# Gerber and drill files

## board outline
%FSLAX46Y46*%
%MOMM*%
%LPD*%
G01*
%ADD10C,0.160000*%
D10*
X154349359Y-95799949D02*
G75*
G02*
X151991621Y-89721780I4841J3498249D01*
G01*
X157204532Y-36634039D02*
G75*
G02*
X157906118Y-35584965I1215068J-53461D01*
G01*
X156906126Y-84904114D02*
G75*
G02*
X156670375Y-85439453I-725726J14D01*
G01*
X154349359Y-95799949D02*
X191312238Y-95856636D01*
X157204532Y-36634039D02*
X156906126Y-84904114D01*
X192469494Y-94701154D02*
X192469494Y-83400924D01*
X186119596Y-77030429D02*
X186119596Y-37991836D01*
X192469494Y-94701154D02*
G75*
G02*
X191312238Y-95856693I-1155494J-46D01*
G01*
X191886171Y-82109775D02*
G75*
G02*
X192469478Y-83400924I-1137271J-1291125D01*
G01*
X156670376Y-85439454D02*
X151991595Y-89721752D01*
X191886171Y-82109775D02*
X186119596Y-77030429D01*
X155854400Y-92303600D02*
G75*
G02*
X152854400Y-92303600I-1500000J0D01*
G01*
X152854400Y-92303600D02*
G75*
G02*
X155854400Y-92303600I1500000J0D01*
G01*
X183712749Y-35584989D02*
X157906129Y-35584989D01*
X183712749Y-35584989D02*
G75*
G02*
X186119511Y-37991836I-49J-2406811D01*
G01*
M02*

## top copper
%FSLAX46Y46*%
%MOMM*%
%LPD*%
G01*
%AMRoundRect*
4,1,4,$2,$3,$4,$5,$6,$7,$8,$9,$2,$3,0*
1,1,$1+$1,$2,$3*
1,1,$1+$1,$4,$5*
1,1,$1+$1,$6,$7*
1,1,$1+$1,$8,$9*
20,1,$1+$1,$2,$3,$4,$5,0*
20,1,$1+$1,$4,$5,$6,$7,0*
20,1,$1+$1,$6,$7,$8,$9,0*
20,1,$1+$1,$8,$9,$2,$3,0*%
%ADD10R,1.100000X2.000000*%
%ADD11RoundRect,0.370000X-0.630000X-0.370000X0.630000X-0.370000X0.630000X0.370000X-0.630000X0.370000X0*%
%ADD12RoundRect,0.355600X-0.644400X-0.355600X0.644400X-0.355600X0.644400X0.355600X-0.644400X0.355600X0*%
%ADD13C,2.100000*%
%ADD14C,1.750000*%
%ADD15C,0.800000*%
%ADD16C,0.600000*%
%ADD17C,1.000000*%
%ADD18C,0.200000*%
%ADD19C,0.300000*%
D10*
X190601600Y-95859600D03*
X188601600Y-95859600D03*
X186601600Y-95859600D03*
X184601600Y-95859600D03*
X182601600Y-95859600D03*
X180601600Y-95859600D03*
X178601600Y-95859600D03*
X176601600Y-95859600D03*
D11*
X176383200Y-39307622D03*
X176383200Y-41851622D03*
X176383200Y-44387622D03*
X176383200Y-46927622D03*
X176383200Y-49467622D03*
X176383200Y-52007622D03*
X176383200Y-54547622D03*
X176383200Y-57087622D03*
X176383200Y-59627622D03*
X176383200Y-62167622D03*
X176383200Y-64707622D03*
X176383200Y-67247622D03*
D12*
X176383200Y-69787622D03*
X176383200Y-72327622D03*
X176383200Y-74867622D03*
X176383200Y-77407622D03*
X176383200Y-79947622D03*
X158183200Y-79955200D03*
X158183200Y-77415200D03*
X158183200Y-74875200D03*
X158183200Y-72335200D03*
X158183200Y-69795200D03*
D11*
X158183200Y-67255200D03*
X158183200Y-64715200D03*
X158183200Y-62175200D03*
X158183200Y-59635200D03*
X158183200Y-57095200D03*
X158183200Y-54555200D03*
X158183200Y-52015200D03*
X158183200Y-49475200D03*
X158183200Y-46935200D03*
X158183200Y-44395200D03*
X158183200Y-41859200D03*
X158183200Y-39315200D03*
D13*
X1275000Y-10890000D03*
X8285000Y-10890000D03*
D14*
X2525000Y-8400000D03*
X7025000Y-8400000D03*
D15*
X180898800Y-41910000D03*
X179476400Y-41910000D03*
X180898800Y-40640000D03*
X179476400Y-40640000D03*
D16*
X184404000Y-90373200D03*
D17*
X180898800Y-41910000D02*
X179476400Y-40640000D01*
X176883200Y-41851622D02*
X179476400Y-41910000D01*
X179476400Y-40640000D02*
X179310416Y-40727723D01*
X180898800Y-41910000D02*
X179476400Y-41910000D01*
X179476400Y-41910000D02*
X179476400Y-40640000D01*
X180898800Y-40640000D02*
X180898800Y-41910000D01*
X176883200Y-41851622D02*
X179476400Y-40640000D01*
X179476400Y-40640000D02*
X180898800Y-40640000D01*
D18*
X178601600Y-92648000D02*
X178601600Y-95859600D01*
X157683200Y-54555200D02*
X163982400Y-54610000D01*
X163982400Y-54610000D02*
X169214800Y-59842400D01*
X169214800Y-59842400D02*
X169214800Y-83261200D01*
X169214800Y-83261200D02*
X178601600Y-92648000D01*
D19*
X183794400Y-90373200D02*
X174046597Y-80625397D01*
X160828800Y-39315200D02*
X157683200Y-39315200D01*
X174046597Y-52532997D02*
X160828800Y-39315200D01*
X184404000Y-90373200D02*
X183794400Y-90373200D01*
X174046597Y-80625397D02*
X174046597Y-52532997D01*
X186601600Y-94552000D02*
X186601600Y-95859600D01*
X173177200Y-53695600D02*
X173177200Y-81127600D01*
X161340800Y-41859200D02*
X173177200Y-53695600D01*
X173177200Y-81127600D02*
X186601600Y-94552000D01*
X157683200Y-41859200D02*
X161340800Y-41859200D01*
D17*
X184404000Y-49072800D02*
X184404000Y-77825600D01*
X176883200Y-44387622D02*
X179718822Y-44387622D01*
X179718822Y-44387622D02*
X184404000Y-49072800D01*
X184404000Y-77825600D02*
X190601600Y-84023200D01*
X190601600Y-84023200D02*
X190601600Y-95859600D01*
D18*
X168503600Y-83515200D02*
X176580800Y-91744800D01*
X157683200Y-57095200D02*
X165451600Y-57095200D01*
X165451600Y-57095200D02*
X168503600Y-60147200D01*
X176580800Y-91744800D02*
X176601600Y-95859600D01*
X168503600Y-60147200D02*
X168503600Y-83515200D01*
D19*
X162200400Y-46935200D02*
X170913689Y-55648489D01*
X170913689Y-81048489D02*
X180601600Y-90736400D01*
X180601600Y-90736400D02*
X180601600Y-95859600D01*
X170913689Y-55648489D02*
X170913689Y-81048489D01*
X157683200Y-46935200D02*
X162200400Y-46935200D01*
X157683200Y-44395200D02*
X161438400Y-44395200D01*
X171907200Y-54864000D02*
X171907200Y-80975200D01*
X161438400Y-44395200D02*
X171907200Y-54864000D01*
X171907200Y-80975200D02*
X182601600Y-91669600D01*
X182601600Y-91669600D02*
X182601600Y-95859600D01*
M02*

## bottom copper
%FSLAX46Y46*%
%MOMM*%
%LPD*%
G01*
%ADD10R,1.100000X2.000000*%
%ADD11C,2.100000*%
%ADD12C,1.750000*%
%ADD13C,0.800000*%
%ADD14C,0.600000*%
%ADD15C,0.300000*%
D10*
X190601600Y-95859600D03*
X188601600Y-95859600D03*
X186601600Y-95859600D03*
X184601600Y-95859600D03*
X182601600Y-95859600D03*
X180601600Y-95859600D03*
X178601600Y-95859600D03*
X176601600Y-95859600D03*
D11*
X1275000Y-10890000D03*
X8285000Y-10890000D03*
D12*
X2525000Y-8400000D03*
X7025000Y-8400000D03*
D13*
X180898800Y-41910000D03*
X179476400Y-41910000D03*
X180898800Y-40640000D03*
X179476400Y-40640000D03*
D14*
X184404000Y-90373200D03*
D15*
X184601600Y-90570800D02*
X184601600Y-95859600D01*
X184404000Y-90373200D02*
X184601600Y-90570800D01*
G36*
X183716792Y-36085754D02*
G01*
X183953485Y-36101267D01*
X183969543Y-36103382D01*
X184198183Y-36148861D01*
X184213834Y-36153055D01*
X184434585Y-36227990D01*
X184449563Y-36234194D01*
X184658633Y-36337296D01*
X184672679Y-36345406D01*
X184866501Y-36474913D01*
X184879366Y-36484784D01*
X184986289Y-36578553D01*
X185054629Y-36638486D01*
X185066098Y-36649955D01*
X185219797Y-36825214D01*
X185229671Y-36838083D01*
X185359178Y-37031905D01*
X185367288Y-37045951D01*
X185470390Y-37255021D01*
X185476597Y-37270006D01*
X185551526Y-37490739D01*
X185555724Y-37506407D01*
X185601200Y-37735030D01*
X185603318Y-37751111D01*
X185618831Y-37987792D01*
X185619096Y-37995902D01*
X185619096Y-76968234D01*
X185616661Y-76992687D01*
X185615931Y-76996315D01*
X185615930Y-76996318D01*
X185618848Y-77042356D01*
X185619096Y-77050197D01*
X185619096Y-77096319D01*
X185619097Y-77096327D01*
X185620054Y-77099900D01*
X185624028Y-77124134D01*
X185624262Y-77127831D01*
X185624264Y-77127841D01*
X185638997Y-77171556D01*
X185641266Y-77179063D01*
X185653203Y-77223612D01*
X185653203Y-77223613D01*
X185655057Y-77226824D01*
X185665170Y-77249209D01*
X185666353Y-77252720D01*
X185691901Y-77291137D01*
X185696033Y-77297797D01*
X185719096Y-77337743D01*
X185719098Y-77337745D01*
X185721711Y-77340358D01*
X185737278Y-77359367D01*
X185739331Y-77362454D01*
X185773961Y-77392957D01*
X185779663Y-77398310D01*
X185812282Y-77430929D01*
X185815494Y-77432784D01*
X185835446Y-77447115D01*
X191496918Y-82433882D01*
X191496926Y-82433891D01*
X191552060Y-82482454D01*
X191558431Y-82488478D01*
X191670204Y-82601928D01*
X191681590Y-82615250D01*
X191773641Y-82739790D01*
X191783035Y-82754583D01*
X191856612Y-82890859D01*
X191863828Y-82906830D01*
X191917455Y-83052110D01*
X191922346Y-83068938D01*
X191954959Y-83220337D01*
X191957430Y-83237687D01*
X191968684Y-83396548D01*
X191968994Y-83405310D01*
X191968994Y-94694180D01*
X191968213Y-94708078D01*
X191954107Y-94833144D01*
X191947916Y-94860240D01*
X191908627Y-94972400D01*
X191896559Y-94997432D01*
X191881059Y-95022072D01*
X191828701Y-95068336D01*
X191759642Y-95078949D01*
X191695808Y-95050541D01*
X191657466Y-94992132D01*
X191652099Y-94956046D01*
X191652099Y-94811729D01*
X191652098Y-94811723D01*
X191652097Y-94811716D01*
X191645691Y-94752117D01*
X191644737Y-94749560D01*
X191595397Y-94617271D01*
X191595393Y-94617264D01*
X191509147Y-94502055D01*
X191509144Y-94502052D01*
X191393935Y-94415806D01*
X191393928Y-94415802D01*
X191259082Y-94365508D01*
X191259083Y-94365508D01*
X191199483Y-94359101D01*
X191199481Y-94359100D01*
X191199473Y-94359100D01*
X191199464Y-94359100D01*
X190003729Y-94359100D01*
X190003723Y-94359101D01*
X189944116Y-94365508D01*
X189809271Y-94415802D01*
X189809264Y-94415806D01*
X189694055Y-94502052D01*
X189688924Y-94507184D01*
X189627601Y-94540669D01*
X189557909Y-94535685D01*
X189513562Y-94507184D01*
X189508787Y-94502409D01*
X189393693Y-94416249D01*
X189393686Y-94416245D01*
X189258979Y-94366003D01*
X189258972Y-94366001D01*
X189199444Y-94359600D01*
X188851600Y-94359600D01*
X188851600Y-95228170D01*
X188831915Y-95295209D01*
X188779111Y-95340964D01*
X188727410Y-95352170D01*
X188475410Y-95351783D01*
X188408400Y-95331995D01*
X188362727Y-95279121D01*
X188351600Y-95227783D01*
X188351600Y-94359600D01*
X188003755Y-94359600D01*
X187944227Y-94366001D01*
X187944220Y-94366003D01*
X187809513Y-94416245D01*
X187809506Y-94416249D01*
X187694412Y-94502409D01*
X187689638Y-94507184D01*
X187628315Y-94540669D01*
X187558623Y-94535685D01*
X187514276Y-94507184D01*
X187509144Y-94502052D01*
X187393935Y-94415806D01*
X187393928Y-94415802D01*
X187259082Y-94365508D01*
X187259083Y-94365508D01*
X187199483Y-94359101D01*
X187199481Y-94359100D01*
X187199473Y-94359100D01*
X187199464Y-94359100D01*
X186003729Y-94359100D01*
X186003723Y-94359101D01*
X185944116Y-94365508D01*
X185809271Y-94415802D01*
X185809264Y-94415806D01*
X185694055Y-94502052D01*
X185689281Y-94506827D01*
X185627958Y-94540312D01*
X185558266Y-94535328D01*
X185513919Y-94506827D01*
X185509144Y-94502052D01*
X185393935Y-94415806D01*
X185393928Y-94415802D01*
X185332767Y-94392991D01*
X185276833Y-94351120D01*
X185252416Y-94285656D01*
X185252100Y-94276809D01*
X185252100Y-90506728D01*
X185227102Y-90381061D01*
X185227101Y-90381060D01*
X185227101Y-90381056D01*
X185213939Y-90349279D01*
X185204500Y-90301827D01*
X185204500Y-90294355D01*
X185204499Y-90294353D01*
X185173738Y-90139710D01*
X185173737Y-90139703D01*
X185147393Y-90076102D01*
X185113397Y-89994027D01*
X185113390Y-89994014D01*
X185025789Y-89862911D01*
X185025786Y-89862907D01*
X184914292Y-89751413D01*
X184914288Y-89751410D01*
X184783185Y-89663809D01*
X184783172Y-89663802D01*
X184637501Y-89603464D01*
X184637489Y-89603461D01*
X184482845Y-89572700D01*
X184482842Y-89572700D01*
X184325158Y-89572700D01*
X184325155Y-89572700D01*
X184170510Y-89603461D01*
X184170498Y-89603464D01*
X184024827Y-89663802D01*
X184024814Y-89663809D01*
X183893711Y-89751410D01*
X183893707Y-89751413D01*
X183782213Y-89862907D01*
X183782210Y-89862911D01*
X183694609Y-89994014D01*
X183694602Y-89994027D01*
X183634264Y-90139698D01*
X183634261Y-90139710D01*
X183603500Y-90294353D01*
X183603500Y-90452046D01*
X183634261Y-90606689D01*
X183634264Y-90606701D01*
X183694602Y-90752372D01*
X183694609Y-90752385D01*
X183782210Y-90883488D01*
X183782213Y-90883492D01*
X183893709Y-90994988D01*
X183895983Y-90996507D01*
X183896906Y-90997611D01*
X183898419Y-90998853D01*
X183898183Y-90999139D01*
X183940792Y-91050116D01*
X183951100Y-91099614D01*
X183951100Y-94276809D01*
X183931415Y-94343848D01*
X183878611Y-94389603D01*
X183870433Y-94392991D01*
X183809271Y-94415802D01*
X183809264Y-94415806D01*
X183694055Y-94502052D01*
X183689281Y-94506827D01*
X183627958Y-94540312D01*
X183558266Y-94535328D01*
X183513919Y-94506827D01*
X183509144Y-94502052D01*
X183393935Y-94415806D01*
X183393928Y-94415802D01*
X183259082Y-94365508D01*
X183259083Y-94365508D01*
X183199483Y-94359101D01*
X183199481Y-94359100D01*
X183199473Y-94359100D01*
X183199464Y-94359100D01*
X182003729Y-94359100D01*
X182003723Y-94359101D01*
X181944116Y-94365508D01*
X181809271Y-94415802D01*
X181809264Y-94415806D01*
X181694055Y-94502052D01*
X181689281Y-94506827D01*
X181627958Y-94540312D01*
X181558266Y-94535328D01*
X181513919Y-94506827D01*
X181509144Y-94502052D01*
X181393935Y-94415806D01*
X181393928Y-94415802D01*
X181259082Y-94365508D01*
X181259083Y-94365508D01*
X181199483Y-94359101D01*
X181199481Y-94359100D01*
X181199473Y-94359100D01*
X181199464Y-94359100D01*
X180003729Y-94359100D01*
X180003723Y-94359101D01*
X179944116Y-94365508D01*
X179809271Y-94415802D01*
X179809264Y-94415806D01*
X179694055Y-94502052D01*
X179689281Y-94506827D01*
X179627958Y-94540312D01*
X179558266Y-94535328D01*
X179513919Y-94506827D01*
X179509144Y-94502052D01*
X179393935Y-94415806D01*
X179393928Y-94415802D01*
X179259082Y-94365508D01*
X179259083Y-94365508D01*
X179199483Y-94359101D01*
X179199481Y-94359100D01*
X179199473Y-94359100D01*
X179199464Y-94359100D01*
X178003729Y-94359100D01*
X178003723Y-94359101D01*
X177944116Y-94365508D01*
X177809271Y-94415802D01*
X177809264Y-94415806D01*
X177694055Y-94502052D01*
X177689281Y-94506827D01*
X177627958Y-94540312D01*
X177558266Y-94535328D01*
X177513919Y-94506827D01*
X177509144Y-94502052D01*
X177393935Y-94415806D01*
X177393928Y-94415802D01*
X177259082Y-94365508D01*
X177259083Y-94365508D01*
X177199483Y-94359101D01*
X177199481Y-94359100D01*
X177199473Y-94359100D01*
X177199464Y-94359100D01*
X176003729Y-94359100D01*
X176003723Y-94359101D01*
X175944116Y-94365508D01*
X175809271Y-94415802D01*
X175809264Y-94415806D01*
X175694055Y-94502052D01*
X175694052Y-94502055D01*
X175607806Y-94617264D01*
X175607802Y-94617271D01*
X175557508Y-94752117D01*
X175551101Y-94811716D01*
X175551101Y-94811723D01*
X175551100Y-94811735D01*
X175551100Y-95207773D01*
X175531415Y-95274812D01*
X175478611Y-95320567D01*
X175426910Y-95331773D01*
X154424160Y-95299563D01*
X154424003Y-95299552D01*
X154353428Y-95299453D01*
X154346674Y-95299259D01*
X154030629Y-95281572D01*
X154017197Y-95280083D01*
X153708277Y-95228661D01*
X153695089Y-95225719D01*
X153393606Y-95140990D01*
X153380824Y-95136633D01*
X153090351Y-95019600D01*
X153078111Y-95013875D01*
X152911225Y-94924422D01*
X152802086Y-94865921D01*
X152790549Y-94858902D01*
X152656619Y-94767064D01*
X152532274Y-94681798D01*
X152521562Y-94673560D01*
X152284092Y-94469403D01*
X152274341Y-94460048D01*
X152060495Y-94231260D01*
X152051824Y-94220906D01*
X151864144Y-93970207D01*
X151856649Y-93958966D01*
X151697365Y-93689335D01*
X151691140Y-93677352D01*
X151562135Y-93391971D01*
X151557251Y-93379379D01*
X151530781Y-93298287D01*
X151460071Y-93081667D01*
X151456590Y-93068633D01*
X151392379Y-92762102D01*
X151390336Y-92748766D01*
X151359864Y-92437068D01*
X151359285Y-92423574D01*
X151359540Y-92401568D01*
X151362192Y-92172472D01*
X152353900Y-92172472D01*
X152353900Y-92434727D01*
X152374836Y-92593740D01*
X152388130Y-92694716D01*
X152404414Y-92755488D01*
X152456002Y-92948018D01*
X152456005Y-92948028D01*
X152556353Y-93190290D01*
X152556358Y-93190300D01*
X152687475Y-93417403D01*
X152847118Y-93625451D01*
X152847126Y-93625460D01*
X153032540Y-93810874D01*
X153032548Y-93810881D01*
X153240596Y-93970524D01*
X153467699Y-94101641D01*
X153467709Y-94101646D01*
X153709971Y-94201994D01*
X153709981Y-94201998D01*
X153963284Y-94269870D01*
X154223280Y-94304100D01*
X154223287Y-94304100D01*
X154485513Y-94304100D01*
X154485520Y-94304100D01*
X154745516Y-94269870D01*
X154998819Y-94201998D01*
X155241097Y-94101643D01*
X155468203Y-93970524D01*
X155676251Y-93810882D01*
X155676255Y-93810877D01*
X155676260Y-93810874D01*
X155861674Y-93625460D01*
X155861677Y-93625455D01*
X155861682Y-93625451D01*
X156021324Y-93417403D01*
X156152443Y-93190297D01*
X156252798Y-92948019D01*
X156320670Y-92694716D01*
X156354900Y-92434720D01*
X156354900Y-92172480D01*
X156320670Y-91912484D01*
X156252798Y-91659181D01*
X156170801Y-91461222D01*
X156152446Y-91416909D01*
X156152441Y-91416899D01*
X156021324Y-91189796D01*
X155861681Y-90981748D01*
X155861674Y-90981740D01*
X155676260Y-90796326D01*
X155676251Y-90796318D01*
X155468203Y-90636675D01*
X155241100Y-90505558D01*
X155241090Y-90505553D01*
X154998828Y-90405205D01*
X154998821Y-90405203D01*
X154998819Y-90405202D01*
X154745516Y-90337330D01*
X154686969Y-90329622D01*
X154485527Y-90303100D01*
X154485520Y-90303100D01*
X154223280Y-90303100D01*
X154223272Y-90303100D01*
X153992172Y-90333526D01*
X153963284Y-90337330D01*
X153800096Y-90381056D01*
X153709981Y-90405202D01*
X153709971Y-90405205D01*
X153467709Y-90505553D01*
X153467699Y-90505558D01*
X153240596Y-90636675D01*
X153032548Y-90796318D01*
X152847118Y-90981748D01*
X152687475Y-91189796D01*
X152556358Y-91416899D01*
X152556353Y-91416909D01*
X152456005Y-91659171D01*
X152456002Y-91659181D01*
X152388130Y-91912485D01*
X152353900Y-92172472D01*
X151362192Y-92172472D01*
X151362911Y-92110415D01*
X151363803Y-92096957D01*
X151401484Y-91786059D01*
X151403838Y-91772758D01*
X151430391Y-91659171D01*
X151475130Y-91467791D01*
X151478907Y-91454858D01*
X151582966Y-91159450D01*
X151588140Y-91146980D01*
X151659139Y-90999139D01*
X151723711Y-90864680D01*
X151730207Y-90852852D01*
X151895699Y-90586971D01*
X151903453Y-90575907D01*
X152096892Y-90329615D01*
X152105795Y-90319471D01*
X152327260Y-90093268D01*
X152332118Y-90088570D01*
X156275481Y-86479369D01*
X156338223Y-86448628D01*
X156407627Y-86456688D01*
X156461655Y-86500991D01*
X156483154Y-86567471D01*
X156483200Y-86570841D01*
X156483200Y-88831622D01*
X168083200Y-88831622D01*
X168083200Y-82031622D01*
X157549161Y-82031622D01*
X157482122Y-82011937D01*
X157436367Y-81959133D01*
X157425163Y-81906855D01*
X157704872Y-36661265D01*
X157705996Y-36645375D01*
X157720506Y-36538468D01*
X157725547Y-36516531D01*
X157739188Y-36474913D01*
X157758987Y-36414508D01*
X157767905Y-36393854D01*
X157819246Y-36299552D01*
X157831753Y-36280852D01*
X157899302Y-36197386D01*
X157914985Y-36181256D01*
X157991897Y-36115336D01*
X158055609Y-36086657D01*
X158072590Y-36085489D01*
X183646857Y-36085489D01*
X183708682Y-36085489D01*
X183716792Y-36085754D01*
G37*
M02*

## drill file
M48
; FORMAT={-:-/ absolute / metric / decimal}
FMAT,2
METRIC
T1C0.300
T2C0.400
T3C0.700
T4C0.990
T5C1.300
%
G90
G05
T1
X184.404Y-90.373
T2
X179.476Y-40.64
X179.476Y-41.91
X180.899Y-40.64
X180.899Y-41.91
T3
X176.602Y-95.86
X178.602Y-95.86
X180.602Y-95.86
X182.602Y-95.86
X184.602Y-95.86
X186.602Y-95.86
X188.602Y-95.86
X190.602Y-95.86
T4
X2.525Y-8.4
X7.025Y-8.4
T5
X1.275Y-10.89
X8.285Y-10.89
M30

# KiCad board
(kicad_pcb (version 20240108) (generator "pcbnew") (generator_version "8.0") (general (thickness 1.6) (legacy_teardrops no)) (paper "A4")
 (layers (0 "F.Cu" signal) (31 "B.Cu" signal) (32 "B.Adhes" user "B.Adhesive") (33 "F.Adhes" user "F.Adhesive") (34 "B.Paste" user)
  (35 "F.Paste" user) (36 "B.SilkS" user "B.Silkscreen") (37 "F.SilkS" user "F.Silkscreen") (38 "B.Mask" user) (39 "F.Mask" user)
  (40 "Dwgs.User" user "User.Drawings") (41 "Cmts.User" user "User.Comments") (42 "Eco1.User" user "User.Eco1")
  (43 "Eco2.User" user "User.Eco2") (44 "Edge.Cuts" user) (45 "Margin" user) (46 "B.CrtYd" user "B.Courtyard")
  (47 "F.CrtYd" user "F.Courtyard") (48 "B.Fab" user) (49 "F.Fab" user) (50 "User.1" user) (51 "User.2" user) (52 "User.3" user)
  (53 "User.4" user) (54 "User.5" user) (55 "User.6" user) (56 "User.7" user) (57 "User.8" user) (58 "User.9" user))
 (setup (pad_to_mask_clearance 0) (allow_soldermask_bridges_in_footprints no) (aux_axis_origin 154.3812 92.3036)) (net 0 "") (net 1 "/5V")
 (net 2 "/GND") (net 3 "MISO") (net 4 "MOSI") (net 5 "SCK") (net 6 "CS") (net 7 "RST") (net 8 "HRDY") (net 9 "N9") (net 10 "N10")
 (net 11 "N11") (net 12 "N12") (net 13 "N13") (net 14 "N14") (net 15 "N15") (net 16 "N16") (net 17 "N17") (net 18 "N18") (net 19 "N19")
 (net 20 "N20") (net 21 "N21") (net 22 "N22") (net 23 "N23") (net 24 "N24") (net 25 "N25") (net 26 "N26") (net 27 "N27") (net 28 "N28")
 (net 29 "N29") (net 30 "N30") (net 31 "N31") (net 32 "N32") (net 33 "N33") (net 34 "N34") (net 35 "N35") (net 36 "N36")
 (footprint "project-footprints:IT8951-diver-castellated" (layer "F.Cu") (at 183.6016 95.8596 180)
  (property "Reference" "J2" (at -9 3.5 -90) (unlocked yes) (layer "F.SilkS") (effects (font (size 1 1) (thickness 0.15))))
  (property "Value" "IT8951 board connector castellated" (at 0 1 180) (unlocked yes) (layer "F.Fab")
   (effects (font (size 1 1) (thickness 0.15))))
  (pad "1" thru_hole rect (at -7 0 180) (size 1.1 2) (drill 0.7) (layers "*.Cu" "*.Mask") (remove_unused_layers no) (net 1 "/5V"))
  (pad "2" thru_hole rect (at -5 0 180) (size 1.1 2) (drill 0.7) (layers "*.Cu" "*.Mask") (remove_unused_layers no) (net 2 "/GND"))
  (pad "3" thru_hole rect (at -3 0 180) (size 1.1 2) (drill 0.7) (layers "*.Cu" "*.Mask") (remove_unused_layers no) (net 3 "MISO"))
  (pad "4" thru_hole rect (at -1 0 180) (size 1.1 2) (drill 0.7) (layers "*.Cu" "*.Mask") (remove_unused_layers no) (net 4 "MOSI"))
  (pad "5" thru_hole rect (at 1 0 180) (size 1.1 2) (drill 0.7) (layers "*.Cu" "*.Mask") (remove_unused_layers no) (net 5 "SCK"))
  (pad "6" thru_hole rect (at 3 0 180) (size 1.1 2) (drill 0.7) (layers "*.Cu" "*.Mask") (remove_unused_layers no) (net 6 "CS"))
  (pad "7" thru_hole rect (at 5 0 180) (size 1.1 2) (drill 0.7) (layers "*.Cu" "*.Mask") (remove_unused_layers no) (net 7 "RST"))
  (pad "8" thru_hole rect (at 7 0 180) (size 1.1 2) (drill 0.7) (layers "*.Cu" "*.Mask") (remove_unused_layers no) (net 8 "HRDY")))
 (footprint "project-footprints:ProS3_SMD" (layer "F.Cu") (at 167.2832 60.831622)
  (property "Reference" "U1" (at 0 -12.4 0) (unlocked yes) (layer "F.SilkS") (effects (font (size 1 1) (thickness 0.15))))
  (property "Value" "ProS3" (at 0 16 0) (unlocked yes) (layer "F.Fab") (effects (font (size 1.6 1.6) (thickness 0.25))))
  (pad "1" smd roundrect (at 9.6 -21.524) (size 2 1.48) (drill (offset -0.5 0)) (layers "F.Cu" "F.Paste" "F.Mask") (roundrect_rratio 0.25)
   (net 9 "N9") (solder_mask_margin 0.0254))
  (pad "2" smd roundrect (at 9.6 -18.98) (size 2 1.48) (drill (offset -0.5 0)) (layers "F.Cu" "F.Paste" "F.Mask") (roundrect_rratio 0.25)
   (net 2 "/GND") (solder_mask_margin 0.0254))
  (pad "3" smd roundrect (at 9.6 -16.444) (size 2 1.48) (drill (offset -0.5 0)) (layers "F.Cu" "F.Paste" "F.Mask") (roundrect_rratio 0.25)
   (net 1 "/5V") (solder_mask_margin 0.0254))
  (pad "4" smd roundrect (at 9.6 -13.904) (size 2 1.48) (drill (offset -0.5 0)) (layers "F.Cu" "F.Paste" "F.Mask") (roundrect_rratio 0.25)
   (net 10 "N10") (solder_mask_margin 0.0254))
  (pad "5" smd roundrect (at 9.6 -11.364) (size 2 1.48) (drill (offset -0.5 0)) (layers "F.Cu" "F.Paste" "F.Mask") (roundrect_rratio 0.25)
   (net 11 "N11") (solder_mask_margin 0.0254))
  (pad "6" smd roundrect (at 9.6 -8.824) (size 2 1.48) (drill (offset -0.5 0)) (layers "F.Cu" "F.Paste" "F.Mask") (roundrect_rratio 0.25)
   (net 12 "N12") (solder_mask_margin 0.0254))
  (pad "7" smd roundrect (at 9.6 -6.284) (size 2 1.48) (drill (offset -0.5 0)) (layers "F.Cu" "F.Paste" "F.Mask") (roundrect_rratio 0.25)
   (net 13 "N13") (solder_mask_margin 0.0254))
  (pad "8" smd roundrect (at 9.6 -3.744) (size 2 1.48) (drill (offset -0.5 0)) (layers "F.Cu" "F.Paste" "F.Mask") (roundrect_rratio 0.25)
   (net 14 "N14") (solder_mask_margin 0.0254))
  (pad "9" smd roundrect (at 9.6 -1.204) (size 2 1.48) (drill (offset -0.5 0)) (layers "F.Cu" "F.Paste" "F.Mask") (roundrect_rratio 0.25)
   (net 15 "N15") (solder_mask_margin 0.0254))
  (pad "10" smd roundrect (at 9.6 1.336) (size 2 1.48) (drill (offset -0.5 0)) (layers "F.Cu" "F.Paste" "F.Mask") (roundrect_rratio 0.25)
   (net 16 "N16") (solder_mask_margin 0.0254))
  (pad "11" smd roundrect (at 9.6 3.876) (size 2 1.48) (drill (offset -0.5 0)) (layers "F.Cu" "F.Paste" "F.Mask") (roundrect_rratio 0.25)
   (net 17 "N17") (solder_mask_margin 0.0254))
  (pad "12" smd roundrect (at 9.6 6.416) (size 2 1.48) (drill (offset -0.5 0)) (layers "F.Cu" "F.Paste" "F.Mask") (roundrect_rratio 0.25)
   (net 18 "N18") (solder_mask_margin 0.0254))
  (pad "13" smd roundrect (at 9.6 8.956) (size 2 1.4224) (drill (offset -0.5 0)) (layers "F.Cu" "F.Paste" "F.Mask") (roundrect_rratio 0.25)
   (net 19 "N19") (solder_mask_margin 0.0254))
  (pad "14" smd roundrect (at 9.6 11.496) (size 2 1.4224) (drill (offset -0.5 0)) (layers "F.Cu" "F.Paste" "F.Mask") (roundrect_rratio 0.25)
   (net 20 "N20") (solder_mask_margin 0.0254))
  (pad "15" smd roundrect (at 9.6 14.036) (size 2 1.4224) (drill (offset -0.5 0)) (layers "F.Cu" "F.Paste" "F.Mask") (roundrect_rratio 0.25)
   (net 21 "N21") (solder_mask_margin 0.0254))
  (pad "16" smd roundrect (at 9.6 16.576) (size 2 1.4224) (drill (offset -0.5 0)) (layers "F.Cu" "F.Paste" "F.Mask") (roundrect_rratio 0.25)
   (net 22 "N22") (solder_mask_margin 0.0254))
  (pad "17" smd roundrect (at 9.6 19.116) (size 2 1.4224) (drill (offset -0.5 0)) (layers "F.Cu" "F.Paste" "F.Mask") (roundrect_rratio 0.25)
   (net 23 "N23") (solder_mask_margin 0.0254))
  (pad "18" smd roundrect (at -9.6 19.123578) (size 2 1.4224) (drill (offset 0.5 0)) (layers "F.Cu" "F.Paste" "F.Mask")
   (roundrect_rratio 0.25) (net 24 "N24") (solder_mask_margin 0.0254))
  (pad "19" smd roundrect (at -9.6 16.583578) (size 2 1.4224) (drill (offset 0.5 0)) (layers "F.Cu" "F.Paste" "F.Mask")
   (roundrect_rratio 0.25) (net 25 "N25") (solder_mask_margin 0.0254))
  (pad "20" smd roundrect (at -9.6 14.043578) (size 2 1.4224) (drill (offset 0.5 0)) (layers "F.Cu" "F.Paste" "F.Mask")
   (roundrect_rratio 0.25) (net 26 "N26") (solder_mask_margin 0.0254))
  (pad "21" smd roundrect (at -9.6 11.503578) (size 2 1.4224) (drill (offset 0.5 0)) (layers "F.Cu" "F.Paste" "F.Mask")
   (roundrect_rratio 0.25) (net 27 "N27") (solder_mask_margin 0.0254))
  (pad "22" smd roundrect (at -9.6 8.963578) (size 2 1.4224) (drill (offset 0.5 0)) (layers "F.Cu" "F.Paste" "F.Mask")
   (roundrect_rratio 0.25) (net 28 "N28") (solder_mask_margin 0.0254))
  (pad "23" smd roundrect (at -9.6 6.423578) (size 2 1.48) (drill (offset 0.5 0)) (layers "F.Cu" "F.Paste" "F.Mask") (roundrect_rratio 0.25)
   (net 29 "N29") (solder_mask_margin 0.0254))
  (pad "24" smd roundrect (at -9.6 3.883578) (size 2 1.48) (drill (offset 0.5 0)) (layers "F.Cu" "F.Paste" "F.Mask") (roundrect_rratio 0.25)
   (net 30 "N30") (solder_mask_margin 0.0254))
  (pad "25" smd roundrect (at -9.6 1.343578) (size 2 1.48) (drill (offset 0.5 0)) (layers "F.Cu" "F.Paste" "F.Mask") (roundrect_rratio 0.25)
   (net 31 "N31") (solder_mask_margin 0.0254))
  (pad "26" smd roundrect (at -9.6 -1.196422) (size 2 1.48) (drill (offset 0.5 0)) (layers "F.Cu" "F.Paste" "F.Mask")
   (roundrect_rratio 0.25) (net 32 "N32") (solder_mask_margin 0.0254))
  (pad "27" smd roundrect (at -9.6 -3.736422) (size 2 1.48) (drill (offset 0.5 0)) (layers "F.Cu" "F.Paste" "F.Mask")
   (roundrect_rratio 0.25) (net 8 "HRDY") (solder_mask_margin 0.0254))
  (pad "28" smd roundrect (at -9.6 -6.276422) (size 2 1.48) (drill (offset 0.5 0)) (layers "F.Cu" "F.Paste" "F.Mask")
   (roundrect_rratio 0.25) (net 7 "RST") (solder_mask_margin 0.0254))
  (pad "29" smd roundrect (at -9.6 -8.816422) (size 2 1.48) (drill (offset 0.5 0)) (layers "F.Cu" "F.Paste" "F.Mask")
   (roundrect_rratio 0.25) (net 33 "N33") (solder_mask_margin 0.0254))
  (pad "30" smd roundrect (at -9.6 -11.356422) (size 2 1.48) (drill (offset 0.5 0)) (layers "F.Cu" "F.Paste" "F.Mask")
   (roundrect_rratio 0.25) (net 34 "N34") (solder_mask_margin 0.0254))
  (pad "31" smd roundrect (at -9.6 -13.896422) (size 2 1.48) (drill (offset 0.5 0)) (layers "F.Cu" "F.Paste" "F.Mask")
   (roundrect_rratio 0.25) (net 6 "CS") (solder_mask_margin 0.0254))
  (pad "32" smd roundrect (at -9.6 -16.436422) (size 2 1.48) (drill (offset 0.5 0)) (layers "F.Cu" "F.Paste" "F.Mask")
   (roundrect_rratio 0.25) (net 5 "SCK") (solder_mask_margin 0.0254))
  (pad "33" smd roundrect (at -9.6 -18.972422) (size 2 1.48) (drill (offset 0.5 0)) (layers "F.Cu" "F.Paste" "F.Mask")
   (roundrect_rratio 0.25) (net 3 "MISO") (solder_mask_margin 0.0254))
  (pad "34" smd roundrect (at -9.6 -21.516422) (size 2 1.48) (drill (offset 0.5 0)) (layers "F.Cu" "F.Paste" "F.Mask")
   (roundrect_rratio 0.25) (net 4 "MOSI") (solder_mask_margin 0.0254))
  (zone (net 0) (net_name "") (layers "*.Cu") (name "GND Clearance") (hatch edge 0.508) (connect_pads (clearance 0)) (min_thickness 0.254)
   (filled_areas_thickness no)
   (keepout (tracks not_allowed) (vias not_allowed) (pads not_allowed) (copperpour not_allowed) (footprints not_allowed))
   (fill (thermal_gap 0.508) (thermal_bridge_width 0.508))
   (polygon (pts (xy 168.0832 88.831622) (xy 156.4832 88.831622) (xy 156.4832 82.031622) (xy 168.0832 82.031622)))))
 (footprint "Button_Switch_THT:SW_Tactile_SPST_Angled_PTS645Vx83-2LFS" (layer "F.Cu") (at 2.525 8.4)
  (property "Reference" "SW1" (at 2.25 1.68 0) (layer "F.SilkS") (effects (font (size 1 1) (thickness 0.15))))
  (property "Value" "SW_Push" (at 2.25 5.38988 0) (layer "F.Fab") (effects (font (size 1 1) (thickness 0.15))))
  (pad "" thru_hole circle (at -1.25 2.49) (size 2.1 2.1) (drill 1.3) (layers "*.Cu" "*.Mask") (remove_unused_layers no))
  (pad "" thru_hole circle (at 5.76 2.49) (size 2.1 2.1) (drill 1.3) (layers "*.Cu" "*.Mask") (remove_unused_layers no))
  (pad "1" thru_hole circle (at 0 0) (size 1.75 1.75) (drill 0.99) (layers "*.Cu" "*.Mask") (remove_unused_layers no) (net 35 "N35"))
  (pad "2" thru_hole circle (at 4.5 0) (size 1.75 1.75) (drill 0.99) (layers "*.Cu" "*.Mask") (remove_unused_layers no) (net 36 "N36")))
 (gr_arc (start 154.349359 95.799949) (mid 151.092729 93.56682) (end 151.991595 89.721752) (stroke (width 0.16) (type solid))
  (layer "Edge.Cuts"))
 (gr_arc (start 157.204532 36.634039) (mid 157.408616 36.011392) (end 157.906129 35.584989) (stroke (width 0.16) (type solid))
  (layer "Edge.Cuts"))
 (gr_arc (start 156.906126 84.904114) (mid 156.844579 85.196589) (end 156.670376 85.439454) (stroke (width 0.16) (type solid))
  (layer "Edge.Cuts"))
 (gr_line (start 154.349359 95.799949) (end 191.312238 95.856636) (stroke (width 0.16) (type solid)) (layer "Edge.Cuts"))
 (gr_line (start 157.204532 36.634039) (end 156.906126 84.904114) (stroke (width 0.16) (type solid)) (layer "Edge.Cuts"))
 (gr_line (start 192.469494 94.701154) (end 192.469494 83.400924) (stroke (width 0.16) (type solid)) (layer "Edge.Cuts"))
 (gr_line (start 186.119596 77.030429) (end 186.119596 37.991836) (stroke (width 0.16) (type solid)) (layer "Edge.Cuts"))
 (gr_arc (start 192.469494 94.701154) (mid 192.130433 95.51883) (end 191.312238 95.856636) (stroke (width 0.16) (type solid))
  (layer "Edge.Cuts"))
 (gr_arc (start 191.886171 82.109775) (mid 192.316896 82.692522) (end 192.469494 83.400924) (stroke (width 0.16) (type solid))
  (layer "Edge.Cuts"))
 (gr_line (start 156.670376 85.439454) (end 151.991595 89.721752) (stroke (width 0.16) (type solid)) (layer "Edge.Cuts"))
 (gr_line (start 191.886171 82.109775) (end 186.119596 77.030429) (stroke (width 0.16) (type solid)) (layer "Edge.Cuts"))
 (gr_circle (center 154.3544 92.3036) (end 152.8544 92.3036) (stroke (width 0.16) (type solid)) (fill none) (layer "Edge.Cuts"))
 (gr_line (start 183.712749 35.584989) (end 157.906129 35.584989) (stroke (width 0.16) (type solid)) (layer "Edge.Cuts"))
 (gr_arc (start 183.712749 35.584989) (mid 185.414647 36.289938) (end 186.119596 37.991836) (stroke (width 0.16) (type solid))
  (layer "Edge.Cuts"))
 (segment (start 180.8988 41.91) (end 179.4764 40.64) (width 1) (layer "F.Cu") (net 2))
 (segment (start 176.8832 41.851622) (end 179.4764 41.91) (width 1) (layer "F.Cu") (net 2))
 (segment (start 179.4764 40.64) (end 179.310416 40.727723) (width 1) (layer "F.Cu") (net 2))
 (segment (start 180.8988 41.91) (end 179.4764 41.91) (width 1) (layer "F.Cu") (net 2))
 (segment (start 179.4764 41.91) (end 179.4764 40.64) (width 1) (layer "F.Cu") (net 2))
 (segment (start 180.8988 40.64) (end 180.8988 41.91) (width 1) (layer "F.Cu") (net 2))
 (segment (start 176.8832 41.851622) (end 179.4764 40.64) (width 1) (layer "F.Cu") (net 2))
 (segment (start 179.4764 40.64) (end 180.8988 40.64) (width 1) (layer "F.Cu") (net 2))
 (via (at 180.8988 41.91) (size 0.8) (drill 0.4) (layers "F.Cu" "B.Cu") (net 2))
 (via (at 179.4764 41.91) (size 0.8) (drill 0.4) (layers "F.Cu" "B.Cu") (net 2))
 (via (at 180.8988 40.64) (size 0.8) (drill 0.4) (layers "F.Cu" "B.Cu") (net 2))
 (via (at 179.4764 40.64) (size 0.8) (drill 0.4) (layers "F.Cu" "B.Cu") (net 2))
 (segment (start 178.6016 92.648) (end 178.6016 95.8596) (width 0.2) (layer "F.Cu") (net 7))
 (segment (start 157.6832 54.5552) (end 163.9824 54.61) (width 0.2) (layer "F.Cu") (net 7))
 (segment (start 163.9824 54.61) (end 169.2148 59.8424) (width 0.2) (layer "F.Cu") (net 7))
 (segment (start 169.2148 59.8424) (end 169.2148 83.2612) (width 0.2) (layer "F.Cu") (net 7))
 (segment (start 169.2148 83.2612) (end 178.6016 92.648) (width 0.2) (layer "F.Cu") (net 7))
 (segment (start 183.7944 90.3732) (end 174.046597 80.625397) (width 0.3) (layer "F.Cu") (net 4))
 (segment (start 160.8288 39.3152) (end 157.6832 39.3152) (width 0.3) (layer "F.Cu") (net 4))
 (segment (start 174.046597 52.532997) (end 160.8288 39.3152) (width 0.3) (layer "F.Cu") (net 4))
 (segment (start 184.404 90.3732) (end 183.7944 90.3732) (width 0.3) (layer "F.Cu") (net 4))
 (segment (start 174.046597 80.625397) (end 174.046597 52.532997) (width 0.3) (layer "F.Cu") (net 4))
 (via (at 184.404 90.3732) (size 0.6) (drill 0.3) (layers "F.Cu" "B.Cu") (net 4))
 (segment (start 184.6016 90.5708) (end 184.6016 95.8596) (width 0.3) (layer "B.Cu") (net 4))
 (segment (start 184.404 90.3732) (end 184.6016 90.5708) (width 0.3) (layer "B.Cu") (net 4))
 (segment (start 186.6016 94.552) (end 186.6016 95.8596) (width 0.3) (layer "F.Cu") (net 3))
 (segment (start 173.1772 53.6956) (end 173.1772 81.1276) (width 0.3) (layer "F.Cu") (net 3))
 (segment (start 161.3408 41.8592) (end 173.1772 53.6956) (width 0.3) (layer "F.Cu") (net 3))
 (segment (start 173.1772 81.1276) (end 186.6016 94.552) (width 0.3) (layer "F.Cu") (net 3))
 (segment (start 157.6832 41.8592) (end 161.3408 41.8592) (width 0.3) (layer "F.Cu") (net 3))
 (segment (start 184.404 49.0728) (end 184.404 77.8256) (width 1) (layer "F.Cu") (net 1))
 (segment (start 176.8832 44.387622) (end 179.718822 44.387622) (width 1) (layer "F.Cu") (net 1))
 (segment (start 179.718822 44.387622) (end 184.404 49.0728) (width 1) (layer "F.Cu") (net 1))
 (segment (start 184.404 77.8256) (end 190.6016 84.0232) (width 1) (layer "F.Cu") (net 1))
 (segment (start 190.6016 84.0232) (end 190.6016 95.8596) (width 1) (layer "F.Cu") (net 1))
 (segment (start 168.5036 83.5152) (end 176.5808 91.7448) (width 0.2) (layer "F.Cu") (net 8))
 (segment (start 157.6832 57.0952) (end 165.4516 57.0952) (width 0.2) (layer "F.Cu") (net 8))
 (segment (start 165.4516 57.0952) (end 168.5036 60.1472) (width 0.2) (layer "F.Cu") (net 8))
 (segment (start 176.5808 91.7448) (end 176.6016 95.8596) (width 0.2) (layer "F.Cu") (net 8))
 (segment (start 168.5036 60.1472) (end 168.5036 83.5152) (width 0.2) (layer "F.Cu") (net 8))
 (segment (start 162.2004 46.9352) (end 170.913689 55.648489) (width 0.3) (layer "F.Cu") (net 6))
 (segment (start 170.913689 81.048489) (end 180.6016 90.7364) (width 0.3) (layer "F.Cu") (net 6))
 (segment (start 180.6016 90.7364) (end 180.6016 95.8596) (width 0.3) (layer "F.Cu") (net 6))
 (segment (start 170.913689 55.648489) (end 170.913689 81.048489) (width 0.3) (layer "F.Cu") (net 6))
 (segment (start 157.6832 46.9352) (end 162.2004 46.9352) (width 0.3) (layer "F.Cu") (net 6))
 (segment (start 157.6832 44.3952) (end 161.4384 44.3952) (width 0.3) (layer "F.Cu") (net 5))
 (segment (start 171.9072 54.864) (end 171.9072 80.9752) (width 0.3) (layer "F.Cu") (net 5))
 (segment (start 161.4384 44.3952) (end 171.9072 54.864) (width 0.3) (layer "F.Cu") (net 5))
 (segment (start 171.9072 80.9752) (end 182.6016 91.6696) (width 0.3) (layer "F.Cu") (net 5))
 (segment (start 182.6016 91.6696) (end 182.6016 95.8596) (width 0.3) (layer "F.Cu") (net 5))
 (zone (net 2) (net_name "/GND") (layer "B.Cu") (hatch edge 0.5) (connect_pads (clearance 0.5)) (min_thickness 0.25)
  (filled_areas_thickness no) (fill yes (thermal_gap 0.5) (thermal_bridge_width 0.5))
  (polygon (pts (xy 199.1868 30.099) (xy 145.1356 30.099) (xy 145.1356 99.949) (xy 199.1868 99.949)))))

